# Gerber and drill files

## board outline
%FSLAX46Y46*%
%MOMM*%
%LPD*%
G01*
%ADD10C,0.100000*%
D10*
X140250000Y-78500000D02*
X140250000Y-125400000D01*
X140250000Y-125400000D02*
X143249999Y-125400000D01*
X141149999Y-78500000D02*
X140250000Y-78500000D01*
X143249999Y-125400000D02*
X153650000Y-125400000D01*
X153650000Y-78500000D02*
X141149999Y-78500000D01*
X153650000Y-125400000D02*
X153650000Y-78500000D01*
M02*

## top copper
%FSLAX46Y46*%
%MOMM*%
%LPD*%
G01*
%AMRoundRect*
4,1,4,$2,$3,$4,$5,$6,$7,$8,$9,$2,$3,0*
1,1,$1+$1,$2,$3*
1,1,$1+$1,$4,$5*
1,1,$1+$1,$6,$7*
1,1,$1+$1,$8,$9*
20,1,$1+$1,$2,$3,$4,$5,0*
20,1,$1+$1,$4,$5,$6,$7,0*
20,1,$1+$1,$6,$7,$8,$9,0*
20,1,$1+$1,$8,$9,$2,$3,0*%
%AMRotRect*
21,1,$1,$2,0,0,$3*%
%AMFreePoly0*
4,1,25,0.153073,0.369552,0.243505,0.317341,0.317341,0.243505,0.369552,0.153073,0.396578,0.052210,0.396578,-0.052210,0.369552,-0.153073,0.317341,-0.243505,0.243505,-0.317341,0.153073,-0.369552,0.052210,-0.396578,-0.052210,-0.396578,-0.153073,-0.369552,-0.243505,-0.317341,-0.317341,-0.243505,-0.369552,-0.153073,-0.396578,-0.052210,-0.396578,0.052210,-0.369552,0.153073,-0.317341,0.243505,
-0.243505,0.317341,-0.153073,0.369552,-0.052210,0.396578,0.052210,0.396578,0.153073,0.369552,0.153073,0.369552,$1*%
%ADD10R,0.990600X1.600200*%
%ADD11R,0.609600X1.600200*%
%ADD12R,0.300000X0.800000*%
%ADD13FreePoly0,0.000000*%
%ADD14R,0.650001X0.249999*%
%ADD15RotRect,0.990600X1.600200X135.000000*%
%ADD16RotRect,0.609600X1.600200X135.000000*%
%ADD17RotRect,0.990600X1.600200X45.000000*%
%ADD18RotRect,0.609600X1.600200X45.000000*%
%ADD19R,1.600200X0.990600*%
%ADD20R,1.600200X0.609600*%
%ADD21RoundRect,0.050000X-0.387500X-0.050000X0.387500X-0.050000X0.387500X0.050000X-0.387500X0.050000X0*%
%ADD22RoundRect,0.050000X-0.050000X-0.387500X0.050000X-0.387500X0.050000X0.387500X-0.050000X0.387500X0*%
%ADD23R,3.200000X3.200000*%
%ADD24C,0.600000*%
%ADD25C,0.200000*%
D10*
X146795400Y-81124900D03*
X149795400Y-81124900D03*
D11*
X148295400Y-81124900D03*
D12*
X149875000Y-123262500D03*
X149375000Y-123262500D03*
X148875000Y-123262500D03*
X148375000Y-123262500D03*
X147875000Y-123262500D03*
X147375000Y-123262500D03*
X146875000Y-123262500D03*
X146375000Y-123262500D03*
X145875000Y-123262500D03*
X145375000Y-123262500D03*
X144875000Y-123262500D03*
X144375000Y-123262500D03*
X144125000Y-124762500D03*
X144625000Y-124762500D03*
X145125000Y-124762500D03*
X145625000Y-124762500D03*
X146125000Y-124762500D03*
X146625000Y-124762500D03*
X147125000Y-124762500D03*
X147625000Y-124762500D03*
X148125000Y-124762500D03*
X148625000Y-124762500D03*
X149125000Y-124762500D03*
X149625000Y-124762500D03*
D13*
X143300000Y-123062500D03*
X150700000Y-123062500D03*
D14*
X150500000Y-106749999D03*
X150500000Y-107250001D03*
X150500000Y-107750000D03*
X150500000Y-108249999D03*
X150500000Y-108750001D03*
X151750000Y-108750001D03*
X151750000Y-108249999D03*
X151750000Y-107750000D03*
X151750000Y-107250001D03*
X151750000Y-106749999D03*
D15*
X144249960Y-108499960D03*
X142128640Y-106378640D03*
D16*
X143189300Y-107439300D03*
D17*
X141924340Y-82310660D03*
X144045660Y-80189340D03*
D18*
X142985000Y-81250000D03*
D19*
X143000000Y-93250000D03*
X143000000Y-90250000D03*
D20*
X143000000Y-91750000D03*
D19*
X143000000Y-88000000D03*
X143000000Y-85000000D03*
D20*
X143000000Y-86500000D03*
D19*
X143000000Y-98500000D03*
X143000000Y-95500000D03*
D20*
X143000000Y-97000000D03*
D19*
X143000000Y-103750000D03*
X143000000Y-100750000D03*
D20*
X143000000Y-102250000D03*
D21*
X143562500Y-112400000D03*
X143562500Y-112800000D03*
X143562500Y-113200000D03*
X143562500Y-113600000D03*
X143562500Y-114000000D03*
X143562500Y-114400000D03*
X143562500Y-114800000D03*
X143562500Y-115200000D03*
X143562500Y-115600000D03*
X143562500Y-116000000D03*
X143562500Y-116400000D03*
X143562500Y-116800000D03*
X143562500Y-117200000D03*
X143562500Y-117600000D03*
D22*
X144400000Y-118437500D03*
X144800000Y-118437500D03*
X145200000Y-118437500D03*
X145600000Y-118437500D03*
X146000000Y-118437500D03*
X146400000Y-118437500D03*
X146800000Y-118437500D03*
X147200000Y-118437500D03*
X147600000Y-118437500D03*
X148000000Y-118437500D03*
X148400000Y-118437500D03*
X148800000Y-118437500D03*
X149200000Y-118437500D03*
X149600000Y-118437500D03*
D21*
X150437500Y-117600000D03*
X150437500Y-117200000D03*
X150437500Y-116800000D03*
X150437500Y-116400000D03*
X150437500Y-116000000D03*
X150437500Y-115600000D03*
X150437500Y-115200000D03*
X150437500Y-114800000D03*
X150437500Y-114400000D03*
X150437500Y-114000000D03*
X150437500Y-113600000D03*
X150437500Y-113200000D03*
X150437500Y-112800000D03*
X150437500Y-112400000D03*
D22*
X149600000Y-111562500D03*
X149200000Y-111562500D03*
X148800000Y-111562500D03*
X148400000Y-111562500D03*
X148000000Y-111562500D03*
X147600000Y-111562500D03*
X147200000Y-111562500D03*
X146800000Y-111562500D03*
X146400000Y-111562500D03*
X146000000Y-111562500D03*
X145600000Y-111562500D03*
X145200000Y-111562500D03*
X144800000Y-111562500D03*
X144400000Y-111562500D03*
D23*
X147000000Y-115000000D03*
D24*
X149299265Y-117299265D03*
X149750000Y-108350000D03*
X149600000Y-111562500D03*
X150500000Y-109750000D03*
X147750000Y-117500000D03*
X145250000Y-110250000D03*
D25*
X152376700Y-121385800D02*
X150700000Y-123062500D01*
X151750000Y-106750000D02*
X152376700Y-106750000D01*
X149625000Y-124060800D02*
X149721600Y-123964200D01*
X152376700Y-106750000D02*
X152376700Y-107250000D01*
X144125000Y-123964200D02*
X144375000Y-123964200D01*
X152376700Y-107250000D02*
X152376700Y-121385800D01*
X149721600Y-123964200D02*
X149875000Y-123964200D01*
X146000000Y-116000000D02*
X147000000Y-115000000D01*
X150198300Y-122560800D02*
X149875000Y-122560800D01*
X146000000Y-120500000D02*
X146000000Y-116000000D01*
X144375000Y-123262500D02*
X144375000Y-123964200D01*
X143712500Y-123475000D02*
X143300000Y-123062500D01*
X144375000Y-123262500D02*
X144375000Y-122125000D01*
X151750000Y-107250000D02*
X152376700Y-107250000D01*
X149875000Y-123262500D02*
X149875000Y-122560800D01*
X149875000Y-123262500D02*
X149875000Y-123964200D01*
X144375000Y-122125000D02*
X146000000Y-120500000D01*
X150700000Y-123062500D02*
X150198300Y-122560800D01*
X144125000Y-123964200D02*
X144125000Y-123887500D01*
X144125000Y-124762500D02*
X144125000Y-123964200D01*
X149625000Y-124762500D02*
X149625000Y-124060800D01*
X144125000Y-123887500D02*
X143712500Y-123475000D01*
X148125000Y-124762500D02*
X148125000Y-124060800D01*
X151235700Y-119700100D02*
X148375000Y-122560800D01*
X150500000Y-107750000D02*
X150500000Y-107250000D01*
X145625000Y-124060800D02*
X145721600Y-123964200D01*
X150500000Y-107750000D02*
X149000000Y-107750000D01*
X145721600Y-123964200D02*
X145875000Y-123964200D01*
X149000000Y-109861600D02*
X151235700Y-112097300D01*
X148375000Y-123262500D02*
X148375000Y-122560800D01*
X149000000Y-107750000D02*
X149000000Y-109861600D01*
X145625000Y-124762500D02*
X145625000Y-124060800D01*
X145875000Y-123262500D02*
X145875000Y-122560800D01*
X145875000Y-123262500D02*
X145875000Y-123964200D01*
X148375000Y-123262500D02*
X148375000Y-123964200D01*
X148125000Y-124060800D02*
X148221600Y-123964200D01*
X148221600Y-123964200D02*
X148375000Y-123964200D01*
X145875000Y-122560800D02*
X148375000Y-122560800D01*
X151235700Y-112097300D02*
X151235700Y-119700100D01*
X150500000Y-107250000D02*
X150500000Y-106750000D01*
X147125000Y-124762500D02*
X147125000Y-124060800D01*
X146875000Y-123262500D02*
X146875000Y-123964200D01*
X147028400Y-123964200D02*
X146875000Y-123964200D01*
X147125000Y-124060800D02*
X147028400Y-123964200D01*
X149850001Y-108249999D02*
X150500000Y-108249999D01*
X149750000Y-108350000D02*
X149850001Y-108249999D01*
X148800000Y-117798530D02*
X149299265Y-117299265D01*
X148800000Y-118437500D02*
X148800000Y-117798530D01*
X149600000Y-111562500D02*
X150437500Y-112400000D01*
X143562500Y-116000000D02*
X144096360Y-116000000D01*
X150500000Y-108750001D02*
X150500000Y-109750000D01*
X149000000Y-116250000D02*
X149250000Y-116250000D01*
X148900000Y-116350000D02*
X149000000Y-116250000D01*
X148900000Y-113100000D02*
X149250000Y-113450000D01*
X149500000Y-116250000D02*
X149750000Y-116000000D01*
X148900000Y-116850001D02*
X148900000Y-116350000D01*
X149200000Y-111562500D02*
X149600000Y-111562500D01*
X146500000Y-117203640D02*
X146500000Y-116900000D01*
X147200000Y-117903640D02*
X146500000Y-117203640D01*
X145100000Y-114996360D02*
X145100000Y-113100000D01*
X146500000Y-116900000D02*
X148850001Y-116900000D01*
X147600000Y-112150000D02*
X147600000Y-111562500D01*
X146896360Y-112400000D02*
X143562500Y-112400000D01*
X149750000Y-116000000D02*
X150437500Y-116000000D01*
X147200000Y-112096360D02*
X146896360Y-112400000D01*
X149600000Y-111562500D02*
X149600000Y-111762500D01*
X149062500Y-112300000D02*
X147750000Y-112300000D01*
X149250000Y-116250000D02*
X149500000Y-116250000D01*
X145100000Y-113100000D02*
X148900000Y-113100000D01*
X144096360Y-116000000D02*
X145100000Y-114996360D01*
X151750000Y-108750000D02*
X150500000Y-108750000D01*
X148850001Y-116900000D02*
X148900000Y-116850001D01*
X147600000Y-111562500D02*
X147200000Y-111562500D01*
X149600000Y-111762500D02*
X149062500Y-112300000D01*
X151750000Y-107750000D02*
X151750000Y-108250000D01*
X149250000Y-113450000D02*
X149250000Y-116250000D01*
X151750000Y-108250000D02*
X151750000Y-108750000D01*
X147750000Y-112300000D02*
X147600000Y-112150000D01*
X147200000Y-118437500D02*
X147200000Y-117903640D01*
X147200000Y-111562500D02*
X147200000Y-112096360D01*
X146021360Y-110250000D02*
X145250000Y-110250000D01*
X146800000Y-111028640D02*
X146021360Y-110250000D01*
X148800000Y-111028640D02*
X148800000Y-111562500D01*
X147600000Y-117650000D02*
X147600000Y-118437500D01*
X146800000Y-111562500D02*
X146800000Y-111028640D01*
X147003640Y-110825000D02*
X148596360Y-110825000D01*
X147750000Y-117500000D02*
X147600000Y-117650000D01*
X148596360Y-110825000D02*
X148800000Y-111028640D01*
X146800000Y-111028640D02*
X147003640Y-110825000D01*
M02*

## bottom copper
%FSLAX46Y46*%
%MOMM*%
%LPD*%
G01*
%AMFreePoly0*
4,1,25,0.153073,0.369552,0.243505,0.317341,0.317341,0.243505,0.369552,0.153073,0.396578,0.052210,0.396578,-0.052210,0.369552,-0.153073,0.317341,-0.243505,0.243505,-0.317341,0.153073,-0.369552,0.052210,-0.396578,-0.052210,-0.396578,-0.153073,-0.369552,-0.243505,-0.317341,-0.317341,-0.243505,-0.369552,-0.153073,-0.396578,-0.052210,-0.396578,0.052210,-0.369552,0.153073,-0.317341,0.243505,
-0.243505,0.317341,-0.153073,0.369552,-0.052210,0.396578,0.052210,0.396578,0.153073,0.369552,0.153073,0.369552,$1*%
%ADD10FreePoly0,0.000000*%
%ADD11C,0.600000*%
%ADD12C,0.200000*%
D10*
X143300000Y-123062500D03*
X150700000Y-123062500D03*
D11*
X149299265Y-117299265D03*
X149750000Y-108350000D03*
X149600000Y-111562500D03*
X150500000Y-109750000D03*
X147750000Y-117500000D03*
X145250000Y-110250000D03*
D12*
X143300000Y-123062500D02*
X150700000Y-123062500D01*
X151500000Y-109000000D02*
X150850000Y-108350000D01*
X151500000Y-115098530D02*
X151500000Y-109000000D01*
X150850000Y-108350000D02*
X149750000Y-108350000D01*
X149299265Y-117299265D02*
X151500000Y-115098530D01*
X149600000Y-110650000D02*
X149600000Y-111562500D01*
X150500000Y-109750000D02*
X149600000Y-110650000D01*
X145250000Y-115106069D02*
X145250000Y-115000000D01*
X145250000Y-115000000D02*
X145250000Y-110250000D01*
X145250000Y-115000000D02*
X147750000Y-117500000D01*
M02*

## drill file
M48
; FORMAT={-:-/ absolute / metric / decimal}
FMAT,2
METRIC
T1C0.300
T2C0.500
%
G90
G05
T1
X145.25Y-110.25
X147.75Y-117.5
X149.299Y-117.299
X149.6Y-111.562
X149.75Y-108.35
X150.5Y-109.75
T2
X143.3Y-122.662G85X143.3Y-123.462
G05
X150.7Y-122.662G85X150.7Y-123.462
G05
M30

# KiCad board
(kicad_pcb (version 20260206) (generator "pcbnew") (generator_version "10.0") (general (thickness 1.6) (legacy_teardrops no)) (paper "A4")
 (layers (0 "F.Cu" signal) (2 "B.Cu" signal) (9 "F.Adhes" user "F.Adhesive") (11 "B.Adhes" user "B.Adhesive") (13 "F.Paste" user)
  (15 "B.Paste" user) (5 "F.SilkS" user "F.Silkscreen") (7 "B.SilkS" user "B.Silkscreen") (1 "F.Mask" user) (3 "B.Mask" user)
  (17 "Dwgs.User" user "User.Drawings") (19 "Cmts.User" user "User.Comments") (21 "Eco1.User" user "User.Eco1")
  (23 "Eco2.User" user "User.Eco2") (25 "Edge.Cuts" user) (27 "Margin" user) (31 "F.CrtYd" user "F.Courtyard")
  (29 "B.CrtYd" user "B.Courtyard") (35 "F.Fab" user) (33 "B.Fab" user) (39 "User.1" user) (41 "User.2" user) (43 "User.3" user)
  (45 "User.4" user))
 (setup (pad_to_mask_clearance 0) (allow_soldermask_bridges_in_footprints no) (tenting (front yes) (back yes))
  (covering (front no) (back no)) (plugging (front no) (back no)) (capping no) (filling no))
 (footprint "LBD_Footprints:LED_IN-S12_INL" (layer "F.Cu") (at 148.2954 81.1249)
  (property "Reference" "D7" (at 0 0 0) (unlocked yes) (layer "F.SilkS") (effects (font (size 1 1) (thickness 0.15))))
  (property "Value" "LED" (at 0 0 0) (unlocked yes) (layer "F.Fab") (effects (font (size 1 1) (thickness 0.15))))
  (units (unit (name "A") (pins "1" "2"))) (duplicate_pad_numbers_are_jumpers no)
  (pad "1" smd rect (at -1.5 0) (size 0.9906 1.6002) (layers "F.Cu" "F.Mask" "F.Paste") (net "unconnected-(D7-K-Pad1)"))
  (pad "2" smd rect (at 1.5 0) (size 0.9906 1.6002) (layers "F.Cu" "F.Mask" "F.Paste") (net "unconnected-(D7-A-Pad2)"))
  (pad "3" smd rect (at 0 0) (size 0.6096 1.6002) (layers "F.Cu" "F.Mask")))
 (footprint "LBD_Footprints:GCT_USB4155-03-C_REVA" (layer "F.Cu") (at 147 124.0125)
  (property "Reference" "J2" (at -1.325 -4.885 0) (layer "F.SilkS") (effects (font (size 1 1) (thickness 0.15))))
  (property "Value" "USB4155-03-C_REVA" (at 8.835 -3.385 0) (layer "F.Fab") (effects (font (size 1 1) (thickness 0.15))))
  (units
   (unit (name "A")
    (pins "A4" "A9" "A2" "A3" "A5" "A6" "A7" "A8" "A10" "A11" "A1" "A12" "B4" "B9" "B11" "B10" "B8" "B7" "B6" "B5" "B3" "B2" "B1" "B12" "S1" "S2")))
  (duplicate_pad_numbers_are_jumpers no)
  (pad "A1" smd rect (at 2.875 -0.75) (size 0.3 0.8) (layers "F.Cu" "F.Mask" "F.Paste") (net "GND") (solder_mask_margin 0.102))
  (pad "A2" smd rect (at 2.375 -0.75) (size 0.3 0.8) (layers "F.Cu" "F.Mask" "F.Paste") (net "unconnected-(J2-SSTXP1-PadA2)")
   (solder_mask_margin 0.102))
  (pad "A3" smd rect (at 1.875 -0.75) (size 0.3 0.8) (layers "F.Cu" "F.Mask" "F.Paste") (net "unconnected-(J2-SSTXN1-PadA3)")
   (solder_mask_margin 0.102))
  (pad "A4" smd rect (at 1.375 -0.75) (size 0.3 0.8) (layers "F.Cu" "F.Mask" "F.Paste") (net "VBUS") (solder_mask_margin 0.102))
  (pad "A5" smd rect (at 0.875 -0.75) (size 0.3 0.8) (layers "F.Cu" "F.Mask" "F.Paste") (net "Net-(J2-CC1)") (solder_mask_margin 0.102))
  (pad "A6" smd rect (at 0.375 -0.75) (size 0.3 0.8) (layers "F.Cu" "F.Mask" "F.Paste") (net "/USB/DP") (solder_mask_margin 0.102))
  (pad "A7" smd rect (at -0.125 -0.75) (size 0.3 0.8) (layers "F.Cu" "F.Mask" "F.Paste") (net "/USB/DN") (solder_mask_margin 0.102))
  (pad "A8" smd rect (at -0.625 -0.75) (size 0.3 0.8) (layers "F.Cu" "F.Mask" "F.Paste") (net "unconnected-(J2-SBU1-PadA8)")
   (solder_mask_margin 0.102))
  (pad "A9" smd rect (at -1.125 -0.75) (size 0.3 0.8) (layers "F.Cu" "F.Mask" "F.Paste") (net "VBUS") (solder_mask_margin 0.102))
  (pad "A10" smd rect (at -1.625 -0.75) (size 0.3 0.8) (layers "F.Cu" "F.Mask" "F.Paste") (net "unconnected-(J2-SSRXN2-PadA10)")
   (solder_mask_margin 0.102))
  (pad "A11" smd rect (at -2.125 -0.75) (size 0.3 0.8) (layers "F.Cu" "F.Mask" "F.Paste") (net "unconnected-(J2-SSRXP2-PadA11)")
   (solder_mask_margin 0.102))
  (pad "A12" smd rect (at -2.625 -0.75) (size 0.3 0.8) (layers "F.Cu" "F.Mask" "F.Paste") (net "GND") (solder_mask_margin 0.102))
  (pad "B1" smd rect (at -2.875 0.75) (size 0.3 0.8) (layers "F.Cu" "F.Mask" "F.Paste") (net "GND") (solder_mask_margin 0.102))
  (pad "B2" smd rect (at -2.375 0.75) (size 0.3 0.8) (layers "F.Cu" "F.Mask" "F.Paste") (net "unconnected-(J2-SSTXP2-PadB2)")
   (solder_mask_margin 0.102))
  (pad "B3" smd rect (at -1.875 0.75) (size 0.3 0.8) (layers "F.Cu" "F.Mask" "F.Paste") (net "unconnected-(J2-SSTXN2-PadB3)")
   (solder_mask_margin 0.102))
  (pad "B4" smd rect (at -1.375 0.75) (size 0.3 0.8) (layers "F.Cu" "F.Mask" "F.Paste") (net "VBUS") (solder_mask_margin 0.102))
  (pad "B5" smd rect (at -0.875 0.75) (size 0.3 0.8) (layers "F.Cu" "F.Mask" "F.Paste") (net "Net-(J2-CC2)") (solder_mask_margin 0.102))
  (pad "B6" smd rect (at -0.375 0.75) (size 0.3 0.8) (layers "F.Cu" "F.Mask" "F.Paste") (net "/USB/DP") (solder_mask_margin 0.102))
  (pad "B7" smd rect (at 0.125 0.75) (size 0.3 0.8) (layers "F.Cu" "F.Mask" "F.Paste") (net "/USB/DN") (solder_mask_margin 0.102))
  (pad "B8" smd rect (at 0.625 0.75) (size 0.3 0.8) (layers "F.Cu" "F.Mask" "F.Paste") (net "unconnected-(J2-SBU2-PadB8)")
   (solder_mask_margin 0.102))
  (pad "B9" smd rect (at 1.125 0.75) (size 0.3 0.8) (layers "F.Cu" "F.Mask" "F.Paste") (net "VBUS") (solder_mask_margin 0.102))
  (pad "B10" smd rect (at 1.625 0.75) (size 0.3 0.8) (layers "F.Cu" "F.Mask" "F.Paste") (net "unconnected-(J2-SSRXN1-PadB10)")
   (solder_mask_margin 0.102))
  (pad "B11" smd rect (at 2.125 0.75) (size 0.3 0.8) (layers "F.Cu" "F.Mask" "F.Paste") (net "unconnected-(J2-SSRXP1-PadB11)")
   (solder_mask_margin 0.102))
  (pad "B12" smd rect (at 2.625 0.75) (size 0.3 0.8) (layers "F.Cu" "F.Mask" "F.Paste") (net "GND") (solder_mask_margin 0.102))
  (pad "S1" thru_hole custom (at -3.7 -0.95) (size 0.8 1.6) (drill oval 0.5 1.3) (layers "*.Cu") (remove_unused_layers no) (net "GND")
   (thermal_bridge_angle 90) (options (clearance outline) (anchor circle)) (primitives))
  (pad "S2" thru_hole custom (at 3.7 -0.95) (size 0.8 1.6) (drill oval 0.5 1.3) (layers "*.Cu") (remove_unused_layers no) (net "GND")
   (thermal_bridge_angle 90) (options (clearance outline) (anchor circle)) (primitives)))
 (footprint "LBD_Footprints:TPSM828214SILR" (layer "F.Cu") (at 151.125 107.75)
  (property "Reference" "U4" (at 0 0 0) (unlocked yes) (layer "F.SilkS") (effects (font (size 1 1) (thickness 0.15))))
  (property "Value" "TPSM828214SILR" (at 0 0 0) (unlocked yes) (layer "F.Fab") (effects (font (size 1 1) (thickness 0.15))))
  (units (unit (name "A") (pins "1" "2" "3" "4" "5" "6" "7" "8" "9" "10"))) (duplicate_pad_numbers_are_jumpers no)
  (pad "1" smd rect (at -0.625 -1.000001) (size 0.650001 0.249999) (layers "F.Cu" "F.Mask" "F.Paste") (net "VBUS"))
  (pad "2" smd rect (at -0.625 -0.499999) (size 0.650001 0.249999) (layers "F.Cu" "F.Mask" "F.Paste") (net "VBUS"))
  (pad "3" smd rect (at -0.625 0) (size 0.650001 0.249999) (layers "F.Cu" "F.Mask" "F.Paste") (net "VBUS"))
  (pad "4" smd rect (at -0.625 0.499999) (size 0.650001 0.249999) (layers "F.Cu" "F.Mask" "F.Paste") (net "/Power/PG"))
  (pad "5" smd rect (at -0.625 1.000001) (size 0.650001 0.249999) (layers "F.Cu" "F.Mask" "F.Paste") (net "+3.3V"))
  (pad "6" smd rect (at 0.625 1.000001) (size 0.650001 0.249999) (layers "F.Cu" "F.Mask" "F.Paste") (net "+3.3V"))
  (pad "7" smd rect (at 0.625 0.499999) (size 0.650001 0.249999) (layers "F.Cu" "F.Mask" "F.Paste") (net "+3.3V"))
  (pad "8" smd rect (at 0.625 0) (size 0.650001 0.249999) (layers "F.Cu" "F.Mask" "F.Paste") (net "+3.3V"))
  (pad "9" smd rect (at 0.625 -0.499999) (size 0.650001 0.249999) (layers "F.Cu" "F.Mask" "F.Paste") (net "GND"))
  (pad "10" smd rect (at 0.625 -1.000001) (size 0.650001 0.249999) (layers "F.Cu" "F.Mask" "F.Paste") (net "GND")))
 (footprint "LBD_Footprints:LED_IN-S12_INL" (layer "F.Cu") (at 143.1893 107.4393 135)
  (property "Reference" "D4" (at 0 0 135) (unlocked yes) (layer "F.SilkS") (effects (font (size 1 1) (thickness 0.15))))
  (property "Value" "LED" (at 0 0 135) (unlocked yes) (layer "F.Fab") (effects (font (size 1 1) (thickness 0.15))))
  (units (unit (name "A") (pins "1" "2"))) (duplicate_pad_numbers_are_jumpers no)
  (pad "1" smd rect (at -1.5 0 135) (size 0.9906 1.6002) (layers "F.Cu" "F.Mask" "F.Paste") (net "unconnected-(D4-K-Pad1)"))
  (pad "2" smd rect (at 1.5 0 135) (size 0.9906 1.6002) (layers "F.Cu" "F.Mask" "F.Paste") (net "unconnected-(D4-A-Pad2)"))
  (pad "3" smd rect (at 0 0 135) (size 0.6096 1.6002) (layers "F.Cu" "F.Mask")))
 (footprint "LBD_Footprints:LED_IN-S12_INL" (layer "F.Cu") (at 142.985 81.25 45)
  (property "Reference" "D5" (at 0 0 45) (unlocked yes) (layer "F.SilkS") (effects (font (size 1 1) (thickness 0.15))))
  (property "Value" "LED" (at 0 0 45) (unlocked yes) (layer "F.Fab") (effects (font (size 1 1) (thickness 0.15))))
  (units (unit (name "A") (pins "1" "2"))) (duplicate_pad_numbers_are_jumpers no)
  (pad "1" smd rect (at -1.5 0 45) (size 0.9906 1.6002) (layers "F.Cu" "F.Mask" "F.Paste") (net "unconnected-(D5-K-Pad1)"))
  (pad "2" smd rect (at 1.5 0 45) (size 0.9906 1.6002) (layers "F.Cu" "F.Mask" "F.Paste") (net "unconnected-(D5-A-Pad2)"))
  (pad "3" smd rect (at 0 0 45) (size 0.6096 1.6002) (layers "F.Cu" "F.Mask")))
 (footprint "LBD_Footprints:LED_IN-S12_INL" (layer "F.Cu") (at 143 91.75 90)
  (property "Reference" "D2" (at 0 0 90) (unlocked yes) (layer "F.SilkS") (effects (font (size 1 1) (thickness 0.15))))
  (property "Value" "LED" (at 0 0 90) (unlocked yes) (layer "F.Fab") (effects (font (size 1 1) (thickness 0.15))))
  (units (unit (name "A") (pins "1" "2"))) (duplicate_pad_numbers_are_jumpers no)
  (pad "1" smd rect (at -1.5 0 90) (size 0.9906 1.6002) (layers "F.Cu" "F.Mask" "F.Paste") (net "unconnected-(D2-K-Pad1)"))
  (pad "2" smd rect (at 1.5 0 90) (size 0.9906 1.6002) (layers "F.Cu" "F.Mask" "F.Paste") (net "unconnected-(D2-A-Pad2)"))
  (pad "3" smd rect (at 0 0 90) (size 0.6096 1.6002) (layers "F.Cu" "F.Mask")))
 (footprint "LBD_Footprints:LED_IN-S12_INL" (layer "F.Cu") (at 143 86.5 90)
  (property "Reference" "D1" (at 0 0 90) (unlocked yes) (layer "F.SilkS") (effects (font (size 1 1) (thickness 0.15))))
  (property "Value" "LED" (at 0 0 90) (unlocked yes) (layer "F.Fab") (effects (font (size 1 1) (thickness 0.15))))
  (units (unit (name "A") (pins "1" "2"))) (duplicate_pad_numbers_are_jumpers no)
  (pad "1" smd rect (at -1.5 0 90) (size 0.9906 1.6002) (layers "F.Cu" "F.Mask" "F.Paste") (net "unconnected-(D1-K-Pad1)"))
  (pad "2" smd rect (at 1.5 0 90) (size 0.9906 1.6002) (layers "F.Cu" "F.Mask" "F.Paste") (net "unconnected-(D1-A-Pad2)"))
  (pad "3" smd rect (at 0 0 90) (size 0.6096 1.6002) (layers "F.Cu" "F.Mask")))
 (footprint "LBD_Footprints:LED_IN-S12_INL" (layer "F.Cu") (at 143 97 90)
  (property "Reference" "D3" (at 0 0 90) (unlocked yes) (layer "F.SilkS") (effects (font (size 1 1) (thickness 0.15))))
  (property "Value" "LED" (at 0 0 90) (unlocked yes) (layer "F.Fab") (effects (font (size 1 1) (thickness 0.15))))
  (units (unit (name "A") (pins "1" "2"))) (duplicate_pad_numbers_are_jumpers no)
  (pad "1" smd rect (at -1.5 0 90) (size 0.9906 1.6002) (layers "F.Cu" "F.Mask" "F.Paste") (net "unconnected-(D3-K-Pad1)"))
  (pad "2" smd rect (at 1.5 0 90) (size 0.9906 1.6002) (layers "F.Cu" "F.Mask" "F.Paste") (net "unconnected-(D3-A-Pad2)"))
  (pad "3" smd rect (at 0 0 90) (size 0.6096 1.6002) (layers "F.Cu" "F.Mask")))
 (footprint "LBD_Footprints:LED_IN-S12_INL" (layer "F.Cu") (at 143 102.25 90)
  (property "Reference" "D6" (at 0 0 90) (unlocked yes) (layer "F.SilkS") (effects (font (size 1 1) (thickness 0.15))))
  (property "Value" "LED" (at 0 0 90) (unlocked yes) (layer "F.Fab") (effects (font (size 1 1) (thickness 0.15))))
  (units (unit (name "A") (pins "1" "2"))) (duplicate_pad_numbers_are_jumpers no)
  (pad "1" smd rect (at -1.5 0 90) (size 0.9906 1.6002) (layers "F.Cu" "F.Mask" "F.Paste") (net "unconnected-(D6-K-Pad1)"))
  (pad "2" smd rect (at 1.5 0 90) (size 0.9906 1.6002) (layers "F.Cu" "F.Mask" "F.Paste") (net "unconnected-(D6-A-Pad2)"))
  (pad "3" smd rect (at 0 0 90) (size 0.6096 1.6002) (layers "F.Cu" "F.Mask")))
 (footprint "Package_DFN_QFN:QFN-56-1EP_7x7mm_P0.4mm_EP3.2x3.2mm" (layer "F.Cu") (at 147 115)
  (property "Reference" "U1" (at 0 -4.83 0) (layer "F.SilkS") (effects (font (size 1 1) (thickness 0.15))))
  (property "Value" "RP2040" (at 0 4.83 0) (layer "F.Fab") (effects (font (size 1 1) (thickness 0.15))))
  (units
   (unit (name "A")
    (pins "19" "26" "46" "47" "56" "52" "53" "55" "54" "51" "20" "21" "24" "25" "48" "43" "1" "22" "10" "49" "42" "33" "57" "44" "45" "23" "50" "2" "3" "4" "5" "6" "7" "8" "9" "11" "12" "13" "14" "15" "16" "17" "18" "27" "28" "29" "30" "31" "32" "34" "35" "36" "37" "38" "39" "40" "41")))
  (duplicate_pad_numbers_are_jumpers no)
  (pad "" smd roundrect (at -0.8 -0.8) (size 1.29 1.29) (layers "F.Paste") (roundrect_rratio 0.193798))
  (pad "" smd roundrect (at -0.8 0.8) (size 1.29 1.29) (layers "F.Paste") (roundrect_rratio 0.193798))
  (pad "" smd roundrect (at 0.8 -0.8) (size 1.29 1.29) (layers "F.Paste") (roundrect_rratio 0.193798))
  (pad "" smd roundrect (at 0.8 0.8) (size 1.29 1.29) (layers "F.Paste") (roundrect_rratio 0.193798))
  (pad "1" smd roundrect (at -3.4375 -2.6) (size 0.875 0.2) (layers "F.Cu" "F.Mask" "F.Paste") (roundrect_rratio 0.25) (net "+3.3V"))
  (pad "2" smd roundrect (at -3.4375 -2.2) (size 0.875 0.2) (layers "F.Cu" "F.Mask" "F.Paste") (roundrect_rratio 0.25)
   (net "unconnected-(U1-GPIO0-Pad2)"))
  (pad "3" smd roundrect (at -3.4375 -1.8) (size 0.875 0.2) (layers "F.Cu" "F.Mask" "F.Paste") (roundrect_rratio 0.25)
   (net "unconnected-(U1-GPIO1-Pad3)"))
  (pad "4" smd roundrect (at -3.4375 -1.4) (size 0.875 0.2) (layers "F.Cu" "F.Mask" "F.Paste") (roundrect_rratio 0.25)
   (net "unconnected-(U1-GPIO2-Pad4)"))
  (pad "5" smd roundrect (at -3.4375 -1) (size 0.875 0.2) (layers "F.Cu" "F.Mask" "F.Paste") (roundrect_rratio 0.25)
   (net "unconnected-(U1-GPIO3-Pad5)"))
  (pad "6" smd roundrect (at -3.4375 -0.6) (size 0.875 0.2) (layers "F.Cu" "F.Mask" "F.Paste") (roundrect_rratio 0.25)
   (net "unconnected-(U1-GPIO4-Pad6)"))
  (pad "7" smd roundrect (at -3.4375 -0.2) (size 0.875 0.2) (layers "F.Cu" "F.Mask" "F.Paste") (roundrect_rratio 0.25)
   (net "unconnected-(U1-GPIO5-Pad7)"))
  (pad "8" smd roundrect (at -3.4375 0.2) (size 0.875 0.2) (layers "F.Cu" "F.Mask" "F.Paste") (roundrect_rratio 0.25)
   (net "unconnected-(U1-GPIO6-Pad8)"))
  (pad "9" smd roundrect (at -3.4375 0.6) (size 0.875 0.2) (layers "F.Cu" "F.Mask" "F.Paste") (roundrect_rratio 0.25)
   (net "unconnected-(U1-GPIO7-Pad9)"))
  (pad "10" smd roundrect (at -3.4375 1) (size 0.875 0.2) (layers "F.Cu" "F.Mask" "F.Paste") (roundrect_rratio 0.25) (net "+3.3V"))
  (pad "11" smd roundrect (at -3.4375 1.4) (size 0.875 0.2) (layers "F.Cu" "F.Mask" "F.Paste") (roundrect_rratio 0.25)
   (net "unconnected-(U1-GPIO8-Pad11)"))
  (pad "12" smd roundrect (at -3.4375 1.8) (size 0.875 0.2) (layers "F.Cu" "F.Mask" "F.Paste") (roundrect_rratio 0.25)
   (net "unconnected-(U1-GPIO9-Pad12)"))
  (pad "13" smd roundrect (at -3.4375 2.2) (size 0.875 0.2) (layers "F.Cu" "F.Mask" "F.Paste") (roundrect_rratio 0.25)
   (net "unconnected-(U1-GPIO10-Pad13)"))
  (pad "14" smd roundrect (at -3.4375 2.6) (size 0.875 0.2) (layers "F.Cu" "F.Mask" "F.Paste") (roundrect_rratio 0.25)
   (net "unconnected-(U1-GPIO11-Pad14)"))
  (pad "15" smd roundrect (at -2.6 3.4375) (size 0.2 0.875) (layers "F.Cu" "F.Mask" "F.Paste") (roundrect_rratio 0.25)
   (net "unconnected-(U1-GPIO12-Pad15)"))
  (pad "16" smd roundrect (at -2.2 3.4375) (size 0.2 0.875) (layers "F.Cu" "F.Mask" "F.Paste") (roundrect_rratio 0.25)
   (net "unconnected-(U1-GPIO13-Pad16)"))
  (pad "17" smd roundrect (at -1.8 3.4375) (size 0.2 0.875) (layers "F.Cu" "F.Mask" "F.Paste") (roundrect_rratio 0.25)
   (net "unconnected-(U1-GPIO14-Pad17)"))
  (pad "18" smd roundrect (at -1.4 3.4375) (size 0.2 0.875) (layers "F.Cu" "F.Mask" "F.Paste") (roundrect_rratio 0.25)
   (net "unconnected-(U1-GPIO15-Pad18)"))
  (pad "19" smd roundrect (at -1 3.4375) (size 0.2 0.875) (layers "F.Cu" "F.Mask" "F.Paste") (roundrect_rratio 0.25) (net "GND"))
  (pad "20" smd roundrect (at -0.6 3.4375) (size 0.2 0.875) (layers "F.Cu" "F.Mask" "F.Paste") (roundrect_rratio 0.25) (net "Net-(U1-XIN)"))
  (pad "21" smd roundrect (at -0.2 3.4375) (size 0.2 0.875) (layers "F.Cu" "F.Mask" "F.Paste") (roundrect_rratio 0.25) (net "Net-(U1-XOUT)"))
  (pad "22" smd roundrect (at 0.2 3.4375) (size 0.2 0.875) (layers "F.Cu" "F.Mask" "F.Paste") (roundrect_rratio 0.25) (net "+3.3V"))
  (pad "23" smd roundrect (at 0.6 3.4375) (size 0.2 0.875) (layers "F.Cu" "F.Mask" "F.Paste") (roundrect_rratio 0.25) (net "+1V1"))
  (pad "24" smd roundrect (at 1 3.4375) (size 0.2 0.875) (layers "F.Cu" "F.Mask" "F.Paste") (roundrect_rratio 0.25) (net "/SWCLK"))
  (pad "25" smd roundrect (at 1.4 3.4375) (size 0.2 0.875) (layers "F.Cu" "F.Mask" "F.Paste") (roundrect_rratio 0.25) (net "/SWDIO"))
  (pad "26" smd roundrect (at 1.8 3.4375) (size 0.2 0.875) (layers "F.Cu" "F.Mask" "F.Paste") (roundrect_rratio 0.25) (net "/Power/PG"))
  (pad "27" smd roundrect (at 2.2 3.4375) (size 0.2 0.875) (layers "F.Cu" "F.Mask" "F.Paste") (roundrect_rratio 0.25)
   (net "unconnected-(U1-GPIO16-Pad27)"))
  (pad "28" smd roundrect (at 2.6 3.4375) (size 0.2 0.875) (layers "F.Cu" "F.Mask" "F.Paste") (roundrect_rratio 0.25)
   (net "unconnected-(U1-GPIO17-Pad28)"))
  (pad "29" smd roundrect (at 3.4375 2.6) (size 0.875 0.2) (layers "F.Cu" "F.Mask" "F.Paste") (roundrect_rratio 0.25)
   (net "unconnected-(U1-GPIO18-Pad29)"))
  (pad "30" smd roundrect (at 3.4375 2.2) (size 0.875 0.2) (layers "F.Cu" "F.Mask" "F.Paste") (roundrect_rratio 0.25)
   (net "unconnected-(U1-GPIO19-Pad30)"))
  (pad "31" smd roundrect (at 3.4375 1.8) (size 0.875 0.2) (layers "F.Cu" "F.Mask" "F.Paste") (roundrect_rratio 0.25)
   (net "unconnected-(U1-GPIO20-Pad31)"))
  (pad "32" smd roundrect (at 3.4375 1.4) (size 0.875 0.2) (layers "F.Cu" "F.Mask" "F.Paste") (roundrect_rratio 0.25)
   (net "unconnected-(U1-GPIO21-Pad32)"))
  (pad "33" smd roundrect (at 3.4375 1) (size 0.875 0.2) (layers "F.Cu" "F.Mask" "F.Paste") (roundrect_rratio 0.25) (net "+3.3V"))
  (pad "34" smd roundrect (at 3.4375 0.6) (size 0.875 0.2) (layers "F.Cu" "F.Mask" "F.Paste") (roundrect_rratio 0.25)
   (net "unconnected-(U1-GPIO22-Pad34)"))
  (pad "35" smd roundrect (at 3.4375 0.2) (size 0.875 0.2) (layers "F.Cu" "F.Mask" "F.Paste") (roundrect_rratio 0.25)
   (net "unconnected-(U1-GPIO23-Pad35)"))
  (pad "36" smd roundrect (at 3.4375 -0.2) (size 0.875 0.2) (layers "F.Cu" "F.Mask" "F.Paste") (roundrect_rratio 0.25)
   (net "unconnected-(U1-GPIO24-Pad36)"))
  (pad "37" smd roundrect (at 3.4375 -0.6) (size 0.875 0.2) (layers "F.Cu" "F.Mask" "F.Paste") (roundrect_rratio 0.25)
   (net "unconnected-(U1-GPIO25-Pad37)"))
  (pad "38" smd roundrect (at 3.4375 -1) (size 0.875 0.2) (layers "F.Cu" "F.Mask" "F.Paste") (roundrect_rratio 0.25)
   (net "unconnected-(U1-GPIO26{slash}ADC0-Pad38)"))
  (pad "39" smd roundrect (at 3.4375 -1.4) (size 0.875 0.2) (layers "F.Cu" "F.Mask" "F.Paste") (roundrect_rratio 0.25)
   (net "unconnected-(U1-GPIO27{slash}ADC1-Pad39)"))
  (pad "40" smd roundrect (at 3.4375 -1.8) (size 0.875 0.2) (layers "F.Cu" "F.Mask" "F.Paste") (roundrect_rratio 0.25)
   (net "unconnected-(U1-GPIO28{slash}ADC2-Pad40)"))
  (pad "41" smd roundrect (at 3.4375 -2.2) (size 0.875 0.2) (layers "F.Cu" "F.Mask" "F.Paste") (roundrect_rratio 0.25)
   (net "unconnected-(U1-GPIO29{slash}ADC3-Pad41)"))
  (pad "42" smd roundrect (at 3.4375 -2.6) (size 0.875 0.2) (layers "F.Cu" "F.Mask" "F.Paste") (roundrect_rratio 0.25) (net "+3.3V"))
  (pad "43" smd roundrect (at 2.6 -3.4375) (size 0.2 0.875) (layers "F.Cu" "F.Mask" "F.Paste") (roundrect_rratio 0.25) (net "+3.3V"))
  (pad "44" smd roundrect (at 2.2 -3.4375) (size 0.2 0.875) (layers "F.Cu" "F.Mask" "F.Paste") (roundrect_rratio 0.25) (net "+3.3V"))
  (pad "45" smd roundrect (at 1.8 -3.4375) (size 0.2 0.875) (layers "F.Cu" "F.Mask" "F.Paste") (roundrect_rratio 0.25) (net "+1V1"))
  (pad "46" smd roundrect (at 1.4 -3.4375) (size 0.2 0.875) (layers "F.Cu" "F.Mask" "F.Paste") (roundrect_rratio 0.25) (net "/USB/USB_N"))
  (pad "47" smd roundrect (at 1 -3.4375) (size 0.2 0.875) (layers "F.Cu" "F.Mask" "F.Paste") (roundrect_rratio 0.25) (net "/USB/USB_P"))
  (pad "48" smd roundrect (at 0.6 -3.4375) (size 0.2 0.875) (layers "F.Cu" "F.Mask" "F.Paste") (roundrect_rratio 0.25) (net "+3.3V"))
  (pad "49" smd roundrect (at 0.2 -3.4375) (size 0.2 0.875) (layers "F.Cu" "F.Mask" "F.Paste") (roundrect_rratio 0.25) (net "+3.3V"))
  (pad "50" smd roundrect (at -0.2 -3.4375) (size 0.2 0.875) (layers "F.Cu" "F.Mask" "F.Paste") (roundrect_rratio 0.25) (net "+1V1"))
  (pad "51" smd roundrect (at -0.6 -3.4375) (size 0.2 0.875) (layers "F.Cu" "F.Mask" "F.Paste") (roundrect_rratio 0.25)
   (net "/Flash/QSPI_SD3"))
  (pad "52" smd roundrect (at -1 -3.4375) (size 0.2 0.875) (layers "F.Cu" "F.Mask" "F.Paste") (roundrect_rratio 0.25)
   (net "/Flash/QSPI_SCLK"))
  (pad "53" smd roundrect (at -1.4 -3.4375) (size 0.2 0.875) (layers "F.Cu" "F.Mask" "F.Paste") (roundrect_rratio 0.25)
   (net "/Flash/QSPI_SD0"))
  (pad "54" smd roundrect (at -1.8 -3.4375) (size 0.2 0.875) (layers "F.Cu" "F.Mask" "F.Paste") (roundrect_rratio 0.25)
   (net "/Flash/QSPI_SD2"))
  (pad "55" smd roundrect (at -2.2 -3.4375) (size 0.2 0.875) (layers "F.Cu" "F.Mask" "F.Paste") (roundrect_rratio 0.25)
   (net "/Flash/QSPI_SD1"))
  (pad "56" smd roundrect (at -2.6 -3.4375) (size 0.2 0.875) (layers "F.Cu" "F.Mask" "F.Paste") (roundrect_rratio 0.25)
   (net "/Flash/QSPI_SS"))
  (pad "57" smd rect (at 0 0) (size 3.2 3.2) (layers "F.Cu" "F.Mask") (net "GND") (zone_connect 2)))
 (gr_line (start 140.25 78.5) (end 140.25 125.4) (stroke (width 0.1) (type default)) (layer "Edge.Cuts"))
 (gr_line (start 140.25 125.4) (end 143.249999 125.4) (stroke (width 0.1) (type default)) (layer "Edge.Cuts"))
 (gr_line (start 141.149999 78.5) (end 140.25 78.5) (stroke (width 0.1) (type default)) (layer "Edge.Cuts"))
 (gr_line (start 143.249999 125.4) (end 153.65 125.4) (stroke (width 0.1) (type default)) (layer "Edge.Cuts"))
 (gr_line (start 153.65 78.5) (end 141.149999 78.5) (stroke (width 0.1) (type default)) (layer "Edge.Cuts"))
 (gr_line (start 153.65 125.4) (end 153.65 78.5) (stroke (width 0.1) (type default)) (layer "Edge.Cuts"))
 (segment (start 152.3767 121.3858) (end 150.7 123.0625) (width 0.2) (layer "F.Cu") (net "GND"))
 (segment (start 151.75 106.75) (end 152.3767 106.75) (width 0.2) (layer "F.Cu") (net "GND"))
 (segment (start 149.625 124.0608) (end 149.7216 123.9642) (width 0.2) (layer "F.Cu") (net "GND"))
 (segment (start 152.3767 106.75) (end 152.3767 107.25) (width 0.2) (layer "F.Cu") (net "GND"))
 (segment (start 144.125 123.9642) (end 144.375 123.9642) (width 0.2) (layer "F.Cu") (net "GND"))
 (segment (start 152.3767 107.25) (end 152.3767 121.3858) (width 0.2) (layer "F.Cu") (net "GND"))
 (segment (start 149.7216 123.9642) (end 149.875 123.9642) (width 0.2) (layer "F.Cu") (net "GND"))
 (segment (start 146 116) (end 147 115) (width 0.2) (layer "F.Cu") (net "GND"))
 (segment (start 150.1983 122.5608) (end 149.875 122.5608) (width 0.2) (layer "F.Cu") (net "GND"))
 (segment (start 146 120.5) (end 146 116) (width 0.2) (layer "F.Cu") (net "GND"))
 (segment (start 144.375 123.2625) (end 144.375 123.9642) (width 0.2) (layer "F.Cu") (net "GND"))
 (segment (start 143.7125 123.475) (end 143.3 123.0625) (width 0.2) (layer "F.Cu") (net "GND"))
 (segment (start 144.375 123.2625) (end 144.375 122.125) (width 0.2) (layer "F.Cu") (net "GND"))
 (segment (start 151.75 107.25) (end 152.3767 107.25) (width 0.2) (layer "F.Cu") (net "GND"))
 (segment (start 149.875 123.2625) (end 149.875 122.5608) (width 0.2) (layer "F.Cu") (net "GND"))
 (segment (start 149.875 123.2625) (end 149.875 123.9642) (width 0.2) (layer "F.Cu") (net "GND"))
 (segment (start 144.375 122.125) (end 146 120.5) (width 0.2) (layer "F.Cu") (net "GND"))
 (segment (start 150.7 123.0625) (end 150.1983 122.5608) (width 0.2) (layer "F.Cu") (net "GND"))
 (segment (start 144.125 123.9642) (end 144.125 123.8875) (width 0.2) (layer "F.Cu") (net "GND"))
 (segment (start 144.125 124.7625) (end 144.125 123.9642) (width 0.2) (layer "F.Cu") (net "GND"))
 (segment (start 149.625 124.7625) (end 149.625 124.0608) (width 0.2) (layer "F.Cu") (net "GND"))
 (segment (start 144.125 123.8875) (end 143.7125 123.475) (width 0.2) (layer "F.Cu") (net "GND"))
 (segment (start 143.3 123.0625) (end 150.7 123.0625) (width 0.2) (layer "B.Cu") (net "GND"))
 (segment (start 148.125 124.7625) (end 148.125 124.0608) (width 0.2) (layer "F.Cu") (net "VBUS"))
 (segment (start 151.2357 119.7001) (end 148.375 122.5608) (width 0.2) (layer "F.Cu") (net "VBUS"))
 (segment (start 150.5 107.75) (end 150.5 107.25) (width 0.2) (layer "F.Cu") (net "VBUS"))
 (segment (start 145.625 124.0608) (end 145.7216 123.9642) (width 0.2) (layer "F.Cu") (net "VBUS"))
 (segment (start 150.5 107.75) (end 149 107.75) (width 0.2) (layer "F.Cu") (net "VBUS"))
 (segment (start 145.7216 123.9642) (end 145.875 123.9642) (width 0.2) (layer "F.Cu") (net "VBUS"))
 (segment (start 149 109.8616) (end 151.2357 112.0973) (width 0.2) (layer "F.Cu") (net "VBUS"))
 (segment (start 148.375 123.2625) (end 148.375 122.5608) (width 0.2) (layer "F.Cu") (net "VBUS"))
 (segment (start 149 107.75) (end 149 109.8616) (width 0.2) (layer "F.Cu") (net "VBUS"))
 (segment (start 145.625 124.7625) (end 145.625 124.0608) (width 0.2) (layer "F.Cu") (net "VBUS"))
 (segment (start 145.875 123.2625) (end 145.875 122.5608) (width 0.2) (layer "F.Cu") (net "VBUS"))
 (segment (start 145.875 123.2625) (end 145.875 123.9642) (width 0.2) (layer "F.Cu") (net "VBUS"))
 (segment (start 148.375 123.2625) (end 148.375 123.9642) (width 0.2) (layer "F.Cu") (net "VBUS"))
 (segment (start 148.125 124.0608) (end 148.2216 123.9642) (width 0.2) (layer "F.Cu") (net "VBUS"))
 (segment (start 148.2216 123.9642) (end 148.375 123.9642) (width 0.2) (layer "F.Cu") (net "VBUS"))
 (segment (start 145.875 122.5608) (end 148.375 122.5608) (width 0.2) (layer "F.Cu") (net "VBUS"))
 (segment (start 151.2357 112.0973) (end 151.2357 119.7001) (width 0.2) (layer "F.Cu") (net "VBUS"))
 (segment (start 150.5 107.25) (end 150.5 106.75) (width 0.2) (layer "F.Cu") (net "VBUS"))
 (segment (start 147.125 124.7625) (end 147.125 124.0608) (width 0.2) (layer "F.Cu") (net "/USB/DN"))
 (segment (start 146.875 123.2625) (end 146.875 123.9642) (width 0.2) (layer "F.Cu") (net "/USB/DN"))
 (segment (start 147.0284 123.9642) (end 146.875 123.9642) (width 0.2) (layer "F.Cu") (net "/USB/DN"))
 (segment (start 147.125 124.0608) (end 147.0284 123.9642) (width 0.2) (layer "F.Cu") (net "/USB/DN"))
 (segment (start 149.850001 108.249999) (end 150.5 108.249999) (width 0.2) (layer "F.Cu") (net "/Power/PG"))
 (segment (start 149.75 108.35) (end 149.850001 108.249999) (width 0.2) (layer "F.Cu") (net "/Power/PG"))
 (segment (start 148.8 117.79853) (end 149.299265 117.299265) (width 0.2) (layer "F.Cu") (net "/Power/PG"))
 (segment (start 148.8 118.4375) (end 148.8 117.79853) (width 0.2) (layer "F.Cu") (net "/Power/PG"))
 (via (at 149.299265 117.299265) (size 0.6) (drill 0.3) (layers "F.Cu" "B.Cu") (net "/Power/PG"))
 (via (at 149.75 108.35) (size 0.6) (drill 0.3) (layers "F.Cu" "B.Cu") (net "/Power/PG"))
 (segment (start 151.5 109) (end 150.85 108.35) (width 0.2) (layer "B.Cu") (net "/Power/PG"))
 (segment (start 151.5 115.09853) (end 151.5 109) (width 0.2) (layer "B.Cu") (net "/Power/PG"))
 (segment (start 150.85 108.35) (end 149.75 108.35) (width 0.2) (layer "B.Cu") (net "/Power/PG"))
 (segment (start 149.299265 117.299265) (end 151.5 115.09853) (width 0.2) (layer "B.Cu") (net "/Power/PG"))
 (segment (start 149.6 111.5625) (end 150.4375 112.4) (width 0.2) (layer "F.Cu") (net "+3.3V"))
 (segment (start 143.5625 116) (end 144.09636 116) (width 0.2) (layer "F.Cu") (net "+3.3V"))
 (segment (start 150.5 108.750001) (end 150.5 109.75) (width 0.2) (layer "F.Cu") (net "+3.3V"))
 (segment (start 149 116.25) (end 149.25 116.25) (width 0.2) (layer "F.Cu") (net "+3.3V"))
 (segment (start 148.9 116.35) (end 149 116.25) (width 0.2) (layer "F.Cu") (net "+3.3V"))
 (segment (start 148.9 113.1) (end 149.25 113.45) (width 0.2) (layer "F.Cu") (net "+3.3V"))
 (segment (start 149.5 116.25) (end 149.75 116) (width 0.2) (layer "F.Cu") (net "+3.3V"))
 (segment (start 148.9 116.850001) (end 148.9 116.35) (width 0.2) (layer "F.Cu") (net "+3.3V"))
 (segment (start 149.2 111.5625) (end 149.6 111.5625) (width 0.2) (layer "F.Cu") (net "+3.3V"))
 (segment (start 146.5 117.20364) (end 146.5 116.9) (width 0.2) (layer "F.Cu") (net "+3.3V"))
 (segment (start 147.2 117.90364) (end 146.5 117.20364) (width 0.2) (layer "F.Cu") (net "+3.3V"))
 (segment (start 145.1 114.99636) (end 145.1 113.1) (width 0.2) (layer "F.Cu") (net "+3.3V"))
 (segment (start 146.5 116.9) (end 148.850001 116.9) (width 0.2) (layer "F.Cu") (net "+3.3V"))
 (segment (start 147.6 112.15) (end 147.6 111.5625) (width 0.2) (layer "F.Cu") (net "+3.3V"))
 (segment (start 146.89636 112.4) (end 143.5625 112.4) (width 0.2) (layer "F.Cu") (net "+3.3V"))
 (segment (start 149.75 116) (end 150.4375 116) (width 0.2) (layer "F.Cu") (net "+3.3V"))
 (segment (start 147.2 112.09636) (end 146.89636 112.4) (width 0.2) (layer "F.Cu") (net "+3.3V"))
 (segment (start 149.6 111.5625) (end 149.6 111.7625) (width 0.2) (layer "F.Cu") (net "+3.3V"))
 (segment (start 149.0625 112.3) (end 147.75 112.3) (width 0.2) (layer "F.Cu") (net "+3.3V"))
 (segment (start 149.25 116.25) (end 149.5 116.25) (width 0.2) (layer "F.Cu") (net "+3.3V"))
 (segment (start 145.1 113.1) (end 148.9 113.1) (width 0.2) (layer "F.Cu") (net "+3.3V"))
 (segment (start 144.09636 116) (end 145.1 114.99636) (width 0.2) (layer "F.Cu") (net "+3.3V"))
 (segment (start 151.75 108.75) (end 150.5 108.75) (width 0.2) (layer "F.Cu") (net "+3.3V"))
 (segment (start 148.850001 116.9) (end 148.9 116.850001) (width 0.2) (layer "F.Cu") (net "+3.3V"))
 (segment (start 147.6 111.5625) (end 147.2 111.5625) (width 0.2) (layer "F.Cu") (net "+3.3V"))
 (segment (start 149.6 111.7625) (end 149.0625 112.3) (width 0.2) (layer "F.Cu") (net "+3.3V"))
 (segment (start 151.75 107.75) (end 151.75 108.25) (width 0.2) (layer "F.Cu") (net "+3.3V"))
 (segment (start 149.25 113.45) (end 149.25 116.25) (width 0.2) (layer "F.Cu") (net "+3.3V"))
 (segment (start 151.75 108.25) (end 151.75 108.75) (width 0.2) (layer "F.Cu") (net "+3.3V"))
 (segment (start 147.75 112.3) (end 147.6 112.15) (width 0.2) (layer "F.Cu") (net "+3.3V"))
 (segment (start 147.2 118.4375) (end 147.2 117.90364) (width 0.2) (layer "F.Cu") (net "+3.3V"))
 (segment (start 147.2 111.5625) (end 147.2 112.09636) (width 0.2) (layer "F.Cu") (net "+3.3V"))
 (via (at 149.6 111.5625) (size 0.6) (drill 0.3) (layers "F.Cu" "B.Cu") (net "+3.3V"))
 (via (at 150.5 109.75) (size 0.6) (drill 0.3) (layers "F.Cu" "B.Cu") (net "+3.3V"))
 (segment (start 149.6 110.65) (end 149.6 111.5625) (width 0.2) (layer "B.Cu") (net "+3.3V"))
 (segment (start 150.5 109.75) (end 149.6 110.65) (width 0.2) (layer "B.Cu") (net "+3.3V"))
 (segment (start 146.02136 110.25) (end 145.25 110.25) (width 0.2) (layer "F.Cu") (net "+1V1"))
 (segment (start 146.8 111.02864) (end 146.02136 110.25) (width 0.2) (layer "F.Cu") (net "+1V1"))
 (segment (start 148.8 111.02864) (end 148.8 111.5625) (width 0.2) (layer "F.Cu") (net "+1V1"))
 (segment (start 147.6 117.65) (end 147.6 118.4375) (width 0.2) (layer "F.Cu") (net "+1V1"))
 (segment (start 146.8 111.5625) (end 146.8 111.02864) (width 0.2) (layer "F.Cu") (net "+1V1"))
 (segment (start 147.00364 110.825) (end 148.59636 110.825) (width 0.2) (layer "F.Cu") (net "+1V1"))
 (segment (start 147.75 117.5) (end 147.6 117.65) (width 0.2) (layer "F.Cu") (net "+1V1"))
 (segment (start 148.59636 110.825) (end 148.8 111.02864) (width 0.2) (layer "F.Cu") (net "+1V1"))
 (segment (start 146.8 111.02864) (end 147.00364 110.825) (width 0.2) (layer "F.Cu") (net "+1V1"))
 (via (at 147.75 117.5) (size 0.6) (drill 0.3) (layers "F.Cu" "B.Cu") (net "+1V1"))
 (via (at 145.25 110.25) (size 0.6) (drill 0.3) (layers "F.Cu" "B.Cu") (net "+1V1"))
 (segment (start 145.25 115.106069) (end 145.25 115) (width 0.2) (layer "B.Cu") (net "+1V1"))
 (segment (start 145.25 115) (end 145.25 110.25) (width 0.2) (layer "B.Cu") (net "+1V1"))
 (segment (start 145.25 115) (end 147.75 117.5) (width 0.2) (layer "B.Cu") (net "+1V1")))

